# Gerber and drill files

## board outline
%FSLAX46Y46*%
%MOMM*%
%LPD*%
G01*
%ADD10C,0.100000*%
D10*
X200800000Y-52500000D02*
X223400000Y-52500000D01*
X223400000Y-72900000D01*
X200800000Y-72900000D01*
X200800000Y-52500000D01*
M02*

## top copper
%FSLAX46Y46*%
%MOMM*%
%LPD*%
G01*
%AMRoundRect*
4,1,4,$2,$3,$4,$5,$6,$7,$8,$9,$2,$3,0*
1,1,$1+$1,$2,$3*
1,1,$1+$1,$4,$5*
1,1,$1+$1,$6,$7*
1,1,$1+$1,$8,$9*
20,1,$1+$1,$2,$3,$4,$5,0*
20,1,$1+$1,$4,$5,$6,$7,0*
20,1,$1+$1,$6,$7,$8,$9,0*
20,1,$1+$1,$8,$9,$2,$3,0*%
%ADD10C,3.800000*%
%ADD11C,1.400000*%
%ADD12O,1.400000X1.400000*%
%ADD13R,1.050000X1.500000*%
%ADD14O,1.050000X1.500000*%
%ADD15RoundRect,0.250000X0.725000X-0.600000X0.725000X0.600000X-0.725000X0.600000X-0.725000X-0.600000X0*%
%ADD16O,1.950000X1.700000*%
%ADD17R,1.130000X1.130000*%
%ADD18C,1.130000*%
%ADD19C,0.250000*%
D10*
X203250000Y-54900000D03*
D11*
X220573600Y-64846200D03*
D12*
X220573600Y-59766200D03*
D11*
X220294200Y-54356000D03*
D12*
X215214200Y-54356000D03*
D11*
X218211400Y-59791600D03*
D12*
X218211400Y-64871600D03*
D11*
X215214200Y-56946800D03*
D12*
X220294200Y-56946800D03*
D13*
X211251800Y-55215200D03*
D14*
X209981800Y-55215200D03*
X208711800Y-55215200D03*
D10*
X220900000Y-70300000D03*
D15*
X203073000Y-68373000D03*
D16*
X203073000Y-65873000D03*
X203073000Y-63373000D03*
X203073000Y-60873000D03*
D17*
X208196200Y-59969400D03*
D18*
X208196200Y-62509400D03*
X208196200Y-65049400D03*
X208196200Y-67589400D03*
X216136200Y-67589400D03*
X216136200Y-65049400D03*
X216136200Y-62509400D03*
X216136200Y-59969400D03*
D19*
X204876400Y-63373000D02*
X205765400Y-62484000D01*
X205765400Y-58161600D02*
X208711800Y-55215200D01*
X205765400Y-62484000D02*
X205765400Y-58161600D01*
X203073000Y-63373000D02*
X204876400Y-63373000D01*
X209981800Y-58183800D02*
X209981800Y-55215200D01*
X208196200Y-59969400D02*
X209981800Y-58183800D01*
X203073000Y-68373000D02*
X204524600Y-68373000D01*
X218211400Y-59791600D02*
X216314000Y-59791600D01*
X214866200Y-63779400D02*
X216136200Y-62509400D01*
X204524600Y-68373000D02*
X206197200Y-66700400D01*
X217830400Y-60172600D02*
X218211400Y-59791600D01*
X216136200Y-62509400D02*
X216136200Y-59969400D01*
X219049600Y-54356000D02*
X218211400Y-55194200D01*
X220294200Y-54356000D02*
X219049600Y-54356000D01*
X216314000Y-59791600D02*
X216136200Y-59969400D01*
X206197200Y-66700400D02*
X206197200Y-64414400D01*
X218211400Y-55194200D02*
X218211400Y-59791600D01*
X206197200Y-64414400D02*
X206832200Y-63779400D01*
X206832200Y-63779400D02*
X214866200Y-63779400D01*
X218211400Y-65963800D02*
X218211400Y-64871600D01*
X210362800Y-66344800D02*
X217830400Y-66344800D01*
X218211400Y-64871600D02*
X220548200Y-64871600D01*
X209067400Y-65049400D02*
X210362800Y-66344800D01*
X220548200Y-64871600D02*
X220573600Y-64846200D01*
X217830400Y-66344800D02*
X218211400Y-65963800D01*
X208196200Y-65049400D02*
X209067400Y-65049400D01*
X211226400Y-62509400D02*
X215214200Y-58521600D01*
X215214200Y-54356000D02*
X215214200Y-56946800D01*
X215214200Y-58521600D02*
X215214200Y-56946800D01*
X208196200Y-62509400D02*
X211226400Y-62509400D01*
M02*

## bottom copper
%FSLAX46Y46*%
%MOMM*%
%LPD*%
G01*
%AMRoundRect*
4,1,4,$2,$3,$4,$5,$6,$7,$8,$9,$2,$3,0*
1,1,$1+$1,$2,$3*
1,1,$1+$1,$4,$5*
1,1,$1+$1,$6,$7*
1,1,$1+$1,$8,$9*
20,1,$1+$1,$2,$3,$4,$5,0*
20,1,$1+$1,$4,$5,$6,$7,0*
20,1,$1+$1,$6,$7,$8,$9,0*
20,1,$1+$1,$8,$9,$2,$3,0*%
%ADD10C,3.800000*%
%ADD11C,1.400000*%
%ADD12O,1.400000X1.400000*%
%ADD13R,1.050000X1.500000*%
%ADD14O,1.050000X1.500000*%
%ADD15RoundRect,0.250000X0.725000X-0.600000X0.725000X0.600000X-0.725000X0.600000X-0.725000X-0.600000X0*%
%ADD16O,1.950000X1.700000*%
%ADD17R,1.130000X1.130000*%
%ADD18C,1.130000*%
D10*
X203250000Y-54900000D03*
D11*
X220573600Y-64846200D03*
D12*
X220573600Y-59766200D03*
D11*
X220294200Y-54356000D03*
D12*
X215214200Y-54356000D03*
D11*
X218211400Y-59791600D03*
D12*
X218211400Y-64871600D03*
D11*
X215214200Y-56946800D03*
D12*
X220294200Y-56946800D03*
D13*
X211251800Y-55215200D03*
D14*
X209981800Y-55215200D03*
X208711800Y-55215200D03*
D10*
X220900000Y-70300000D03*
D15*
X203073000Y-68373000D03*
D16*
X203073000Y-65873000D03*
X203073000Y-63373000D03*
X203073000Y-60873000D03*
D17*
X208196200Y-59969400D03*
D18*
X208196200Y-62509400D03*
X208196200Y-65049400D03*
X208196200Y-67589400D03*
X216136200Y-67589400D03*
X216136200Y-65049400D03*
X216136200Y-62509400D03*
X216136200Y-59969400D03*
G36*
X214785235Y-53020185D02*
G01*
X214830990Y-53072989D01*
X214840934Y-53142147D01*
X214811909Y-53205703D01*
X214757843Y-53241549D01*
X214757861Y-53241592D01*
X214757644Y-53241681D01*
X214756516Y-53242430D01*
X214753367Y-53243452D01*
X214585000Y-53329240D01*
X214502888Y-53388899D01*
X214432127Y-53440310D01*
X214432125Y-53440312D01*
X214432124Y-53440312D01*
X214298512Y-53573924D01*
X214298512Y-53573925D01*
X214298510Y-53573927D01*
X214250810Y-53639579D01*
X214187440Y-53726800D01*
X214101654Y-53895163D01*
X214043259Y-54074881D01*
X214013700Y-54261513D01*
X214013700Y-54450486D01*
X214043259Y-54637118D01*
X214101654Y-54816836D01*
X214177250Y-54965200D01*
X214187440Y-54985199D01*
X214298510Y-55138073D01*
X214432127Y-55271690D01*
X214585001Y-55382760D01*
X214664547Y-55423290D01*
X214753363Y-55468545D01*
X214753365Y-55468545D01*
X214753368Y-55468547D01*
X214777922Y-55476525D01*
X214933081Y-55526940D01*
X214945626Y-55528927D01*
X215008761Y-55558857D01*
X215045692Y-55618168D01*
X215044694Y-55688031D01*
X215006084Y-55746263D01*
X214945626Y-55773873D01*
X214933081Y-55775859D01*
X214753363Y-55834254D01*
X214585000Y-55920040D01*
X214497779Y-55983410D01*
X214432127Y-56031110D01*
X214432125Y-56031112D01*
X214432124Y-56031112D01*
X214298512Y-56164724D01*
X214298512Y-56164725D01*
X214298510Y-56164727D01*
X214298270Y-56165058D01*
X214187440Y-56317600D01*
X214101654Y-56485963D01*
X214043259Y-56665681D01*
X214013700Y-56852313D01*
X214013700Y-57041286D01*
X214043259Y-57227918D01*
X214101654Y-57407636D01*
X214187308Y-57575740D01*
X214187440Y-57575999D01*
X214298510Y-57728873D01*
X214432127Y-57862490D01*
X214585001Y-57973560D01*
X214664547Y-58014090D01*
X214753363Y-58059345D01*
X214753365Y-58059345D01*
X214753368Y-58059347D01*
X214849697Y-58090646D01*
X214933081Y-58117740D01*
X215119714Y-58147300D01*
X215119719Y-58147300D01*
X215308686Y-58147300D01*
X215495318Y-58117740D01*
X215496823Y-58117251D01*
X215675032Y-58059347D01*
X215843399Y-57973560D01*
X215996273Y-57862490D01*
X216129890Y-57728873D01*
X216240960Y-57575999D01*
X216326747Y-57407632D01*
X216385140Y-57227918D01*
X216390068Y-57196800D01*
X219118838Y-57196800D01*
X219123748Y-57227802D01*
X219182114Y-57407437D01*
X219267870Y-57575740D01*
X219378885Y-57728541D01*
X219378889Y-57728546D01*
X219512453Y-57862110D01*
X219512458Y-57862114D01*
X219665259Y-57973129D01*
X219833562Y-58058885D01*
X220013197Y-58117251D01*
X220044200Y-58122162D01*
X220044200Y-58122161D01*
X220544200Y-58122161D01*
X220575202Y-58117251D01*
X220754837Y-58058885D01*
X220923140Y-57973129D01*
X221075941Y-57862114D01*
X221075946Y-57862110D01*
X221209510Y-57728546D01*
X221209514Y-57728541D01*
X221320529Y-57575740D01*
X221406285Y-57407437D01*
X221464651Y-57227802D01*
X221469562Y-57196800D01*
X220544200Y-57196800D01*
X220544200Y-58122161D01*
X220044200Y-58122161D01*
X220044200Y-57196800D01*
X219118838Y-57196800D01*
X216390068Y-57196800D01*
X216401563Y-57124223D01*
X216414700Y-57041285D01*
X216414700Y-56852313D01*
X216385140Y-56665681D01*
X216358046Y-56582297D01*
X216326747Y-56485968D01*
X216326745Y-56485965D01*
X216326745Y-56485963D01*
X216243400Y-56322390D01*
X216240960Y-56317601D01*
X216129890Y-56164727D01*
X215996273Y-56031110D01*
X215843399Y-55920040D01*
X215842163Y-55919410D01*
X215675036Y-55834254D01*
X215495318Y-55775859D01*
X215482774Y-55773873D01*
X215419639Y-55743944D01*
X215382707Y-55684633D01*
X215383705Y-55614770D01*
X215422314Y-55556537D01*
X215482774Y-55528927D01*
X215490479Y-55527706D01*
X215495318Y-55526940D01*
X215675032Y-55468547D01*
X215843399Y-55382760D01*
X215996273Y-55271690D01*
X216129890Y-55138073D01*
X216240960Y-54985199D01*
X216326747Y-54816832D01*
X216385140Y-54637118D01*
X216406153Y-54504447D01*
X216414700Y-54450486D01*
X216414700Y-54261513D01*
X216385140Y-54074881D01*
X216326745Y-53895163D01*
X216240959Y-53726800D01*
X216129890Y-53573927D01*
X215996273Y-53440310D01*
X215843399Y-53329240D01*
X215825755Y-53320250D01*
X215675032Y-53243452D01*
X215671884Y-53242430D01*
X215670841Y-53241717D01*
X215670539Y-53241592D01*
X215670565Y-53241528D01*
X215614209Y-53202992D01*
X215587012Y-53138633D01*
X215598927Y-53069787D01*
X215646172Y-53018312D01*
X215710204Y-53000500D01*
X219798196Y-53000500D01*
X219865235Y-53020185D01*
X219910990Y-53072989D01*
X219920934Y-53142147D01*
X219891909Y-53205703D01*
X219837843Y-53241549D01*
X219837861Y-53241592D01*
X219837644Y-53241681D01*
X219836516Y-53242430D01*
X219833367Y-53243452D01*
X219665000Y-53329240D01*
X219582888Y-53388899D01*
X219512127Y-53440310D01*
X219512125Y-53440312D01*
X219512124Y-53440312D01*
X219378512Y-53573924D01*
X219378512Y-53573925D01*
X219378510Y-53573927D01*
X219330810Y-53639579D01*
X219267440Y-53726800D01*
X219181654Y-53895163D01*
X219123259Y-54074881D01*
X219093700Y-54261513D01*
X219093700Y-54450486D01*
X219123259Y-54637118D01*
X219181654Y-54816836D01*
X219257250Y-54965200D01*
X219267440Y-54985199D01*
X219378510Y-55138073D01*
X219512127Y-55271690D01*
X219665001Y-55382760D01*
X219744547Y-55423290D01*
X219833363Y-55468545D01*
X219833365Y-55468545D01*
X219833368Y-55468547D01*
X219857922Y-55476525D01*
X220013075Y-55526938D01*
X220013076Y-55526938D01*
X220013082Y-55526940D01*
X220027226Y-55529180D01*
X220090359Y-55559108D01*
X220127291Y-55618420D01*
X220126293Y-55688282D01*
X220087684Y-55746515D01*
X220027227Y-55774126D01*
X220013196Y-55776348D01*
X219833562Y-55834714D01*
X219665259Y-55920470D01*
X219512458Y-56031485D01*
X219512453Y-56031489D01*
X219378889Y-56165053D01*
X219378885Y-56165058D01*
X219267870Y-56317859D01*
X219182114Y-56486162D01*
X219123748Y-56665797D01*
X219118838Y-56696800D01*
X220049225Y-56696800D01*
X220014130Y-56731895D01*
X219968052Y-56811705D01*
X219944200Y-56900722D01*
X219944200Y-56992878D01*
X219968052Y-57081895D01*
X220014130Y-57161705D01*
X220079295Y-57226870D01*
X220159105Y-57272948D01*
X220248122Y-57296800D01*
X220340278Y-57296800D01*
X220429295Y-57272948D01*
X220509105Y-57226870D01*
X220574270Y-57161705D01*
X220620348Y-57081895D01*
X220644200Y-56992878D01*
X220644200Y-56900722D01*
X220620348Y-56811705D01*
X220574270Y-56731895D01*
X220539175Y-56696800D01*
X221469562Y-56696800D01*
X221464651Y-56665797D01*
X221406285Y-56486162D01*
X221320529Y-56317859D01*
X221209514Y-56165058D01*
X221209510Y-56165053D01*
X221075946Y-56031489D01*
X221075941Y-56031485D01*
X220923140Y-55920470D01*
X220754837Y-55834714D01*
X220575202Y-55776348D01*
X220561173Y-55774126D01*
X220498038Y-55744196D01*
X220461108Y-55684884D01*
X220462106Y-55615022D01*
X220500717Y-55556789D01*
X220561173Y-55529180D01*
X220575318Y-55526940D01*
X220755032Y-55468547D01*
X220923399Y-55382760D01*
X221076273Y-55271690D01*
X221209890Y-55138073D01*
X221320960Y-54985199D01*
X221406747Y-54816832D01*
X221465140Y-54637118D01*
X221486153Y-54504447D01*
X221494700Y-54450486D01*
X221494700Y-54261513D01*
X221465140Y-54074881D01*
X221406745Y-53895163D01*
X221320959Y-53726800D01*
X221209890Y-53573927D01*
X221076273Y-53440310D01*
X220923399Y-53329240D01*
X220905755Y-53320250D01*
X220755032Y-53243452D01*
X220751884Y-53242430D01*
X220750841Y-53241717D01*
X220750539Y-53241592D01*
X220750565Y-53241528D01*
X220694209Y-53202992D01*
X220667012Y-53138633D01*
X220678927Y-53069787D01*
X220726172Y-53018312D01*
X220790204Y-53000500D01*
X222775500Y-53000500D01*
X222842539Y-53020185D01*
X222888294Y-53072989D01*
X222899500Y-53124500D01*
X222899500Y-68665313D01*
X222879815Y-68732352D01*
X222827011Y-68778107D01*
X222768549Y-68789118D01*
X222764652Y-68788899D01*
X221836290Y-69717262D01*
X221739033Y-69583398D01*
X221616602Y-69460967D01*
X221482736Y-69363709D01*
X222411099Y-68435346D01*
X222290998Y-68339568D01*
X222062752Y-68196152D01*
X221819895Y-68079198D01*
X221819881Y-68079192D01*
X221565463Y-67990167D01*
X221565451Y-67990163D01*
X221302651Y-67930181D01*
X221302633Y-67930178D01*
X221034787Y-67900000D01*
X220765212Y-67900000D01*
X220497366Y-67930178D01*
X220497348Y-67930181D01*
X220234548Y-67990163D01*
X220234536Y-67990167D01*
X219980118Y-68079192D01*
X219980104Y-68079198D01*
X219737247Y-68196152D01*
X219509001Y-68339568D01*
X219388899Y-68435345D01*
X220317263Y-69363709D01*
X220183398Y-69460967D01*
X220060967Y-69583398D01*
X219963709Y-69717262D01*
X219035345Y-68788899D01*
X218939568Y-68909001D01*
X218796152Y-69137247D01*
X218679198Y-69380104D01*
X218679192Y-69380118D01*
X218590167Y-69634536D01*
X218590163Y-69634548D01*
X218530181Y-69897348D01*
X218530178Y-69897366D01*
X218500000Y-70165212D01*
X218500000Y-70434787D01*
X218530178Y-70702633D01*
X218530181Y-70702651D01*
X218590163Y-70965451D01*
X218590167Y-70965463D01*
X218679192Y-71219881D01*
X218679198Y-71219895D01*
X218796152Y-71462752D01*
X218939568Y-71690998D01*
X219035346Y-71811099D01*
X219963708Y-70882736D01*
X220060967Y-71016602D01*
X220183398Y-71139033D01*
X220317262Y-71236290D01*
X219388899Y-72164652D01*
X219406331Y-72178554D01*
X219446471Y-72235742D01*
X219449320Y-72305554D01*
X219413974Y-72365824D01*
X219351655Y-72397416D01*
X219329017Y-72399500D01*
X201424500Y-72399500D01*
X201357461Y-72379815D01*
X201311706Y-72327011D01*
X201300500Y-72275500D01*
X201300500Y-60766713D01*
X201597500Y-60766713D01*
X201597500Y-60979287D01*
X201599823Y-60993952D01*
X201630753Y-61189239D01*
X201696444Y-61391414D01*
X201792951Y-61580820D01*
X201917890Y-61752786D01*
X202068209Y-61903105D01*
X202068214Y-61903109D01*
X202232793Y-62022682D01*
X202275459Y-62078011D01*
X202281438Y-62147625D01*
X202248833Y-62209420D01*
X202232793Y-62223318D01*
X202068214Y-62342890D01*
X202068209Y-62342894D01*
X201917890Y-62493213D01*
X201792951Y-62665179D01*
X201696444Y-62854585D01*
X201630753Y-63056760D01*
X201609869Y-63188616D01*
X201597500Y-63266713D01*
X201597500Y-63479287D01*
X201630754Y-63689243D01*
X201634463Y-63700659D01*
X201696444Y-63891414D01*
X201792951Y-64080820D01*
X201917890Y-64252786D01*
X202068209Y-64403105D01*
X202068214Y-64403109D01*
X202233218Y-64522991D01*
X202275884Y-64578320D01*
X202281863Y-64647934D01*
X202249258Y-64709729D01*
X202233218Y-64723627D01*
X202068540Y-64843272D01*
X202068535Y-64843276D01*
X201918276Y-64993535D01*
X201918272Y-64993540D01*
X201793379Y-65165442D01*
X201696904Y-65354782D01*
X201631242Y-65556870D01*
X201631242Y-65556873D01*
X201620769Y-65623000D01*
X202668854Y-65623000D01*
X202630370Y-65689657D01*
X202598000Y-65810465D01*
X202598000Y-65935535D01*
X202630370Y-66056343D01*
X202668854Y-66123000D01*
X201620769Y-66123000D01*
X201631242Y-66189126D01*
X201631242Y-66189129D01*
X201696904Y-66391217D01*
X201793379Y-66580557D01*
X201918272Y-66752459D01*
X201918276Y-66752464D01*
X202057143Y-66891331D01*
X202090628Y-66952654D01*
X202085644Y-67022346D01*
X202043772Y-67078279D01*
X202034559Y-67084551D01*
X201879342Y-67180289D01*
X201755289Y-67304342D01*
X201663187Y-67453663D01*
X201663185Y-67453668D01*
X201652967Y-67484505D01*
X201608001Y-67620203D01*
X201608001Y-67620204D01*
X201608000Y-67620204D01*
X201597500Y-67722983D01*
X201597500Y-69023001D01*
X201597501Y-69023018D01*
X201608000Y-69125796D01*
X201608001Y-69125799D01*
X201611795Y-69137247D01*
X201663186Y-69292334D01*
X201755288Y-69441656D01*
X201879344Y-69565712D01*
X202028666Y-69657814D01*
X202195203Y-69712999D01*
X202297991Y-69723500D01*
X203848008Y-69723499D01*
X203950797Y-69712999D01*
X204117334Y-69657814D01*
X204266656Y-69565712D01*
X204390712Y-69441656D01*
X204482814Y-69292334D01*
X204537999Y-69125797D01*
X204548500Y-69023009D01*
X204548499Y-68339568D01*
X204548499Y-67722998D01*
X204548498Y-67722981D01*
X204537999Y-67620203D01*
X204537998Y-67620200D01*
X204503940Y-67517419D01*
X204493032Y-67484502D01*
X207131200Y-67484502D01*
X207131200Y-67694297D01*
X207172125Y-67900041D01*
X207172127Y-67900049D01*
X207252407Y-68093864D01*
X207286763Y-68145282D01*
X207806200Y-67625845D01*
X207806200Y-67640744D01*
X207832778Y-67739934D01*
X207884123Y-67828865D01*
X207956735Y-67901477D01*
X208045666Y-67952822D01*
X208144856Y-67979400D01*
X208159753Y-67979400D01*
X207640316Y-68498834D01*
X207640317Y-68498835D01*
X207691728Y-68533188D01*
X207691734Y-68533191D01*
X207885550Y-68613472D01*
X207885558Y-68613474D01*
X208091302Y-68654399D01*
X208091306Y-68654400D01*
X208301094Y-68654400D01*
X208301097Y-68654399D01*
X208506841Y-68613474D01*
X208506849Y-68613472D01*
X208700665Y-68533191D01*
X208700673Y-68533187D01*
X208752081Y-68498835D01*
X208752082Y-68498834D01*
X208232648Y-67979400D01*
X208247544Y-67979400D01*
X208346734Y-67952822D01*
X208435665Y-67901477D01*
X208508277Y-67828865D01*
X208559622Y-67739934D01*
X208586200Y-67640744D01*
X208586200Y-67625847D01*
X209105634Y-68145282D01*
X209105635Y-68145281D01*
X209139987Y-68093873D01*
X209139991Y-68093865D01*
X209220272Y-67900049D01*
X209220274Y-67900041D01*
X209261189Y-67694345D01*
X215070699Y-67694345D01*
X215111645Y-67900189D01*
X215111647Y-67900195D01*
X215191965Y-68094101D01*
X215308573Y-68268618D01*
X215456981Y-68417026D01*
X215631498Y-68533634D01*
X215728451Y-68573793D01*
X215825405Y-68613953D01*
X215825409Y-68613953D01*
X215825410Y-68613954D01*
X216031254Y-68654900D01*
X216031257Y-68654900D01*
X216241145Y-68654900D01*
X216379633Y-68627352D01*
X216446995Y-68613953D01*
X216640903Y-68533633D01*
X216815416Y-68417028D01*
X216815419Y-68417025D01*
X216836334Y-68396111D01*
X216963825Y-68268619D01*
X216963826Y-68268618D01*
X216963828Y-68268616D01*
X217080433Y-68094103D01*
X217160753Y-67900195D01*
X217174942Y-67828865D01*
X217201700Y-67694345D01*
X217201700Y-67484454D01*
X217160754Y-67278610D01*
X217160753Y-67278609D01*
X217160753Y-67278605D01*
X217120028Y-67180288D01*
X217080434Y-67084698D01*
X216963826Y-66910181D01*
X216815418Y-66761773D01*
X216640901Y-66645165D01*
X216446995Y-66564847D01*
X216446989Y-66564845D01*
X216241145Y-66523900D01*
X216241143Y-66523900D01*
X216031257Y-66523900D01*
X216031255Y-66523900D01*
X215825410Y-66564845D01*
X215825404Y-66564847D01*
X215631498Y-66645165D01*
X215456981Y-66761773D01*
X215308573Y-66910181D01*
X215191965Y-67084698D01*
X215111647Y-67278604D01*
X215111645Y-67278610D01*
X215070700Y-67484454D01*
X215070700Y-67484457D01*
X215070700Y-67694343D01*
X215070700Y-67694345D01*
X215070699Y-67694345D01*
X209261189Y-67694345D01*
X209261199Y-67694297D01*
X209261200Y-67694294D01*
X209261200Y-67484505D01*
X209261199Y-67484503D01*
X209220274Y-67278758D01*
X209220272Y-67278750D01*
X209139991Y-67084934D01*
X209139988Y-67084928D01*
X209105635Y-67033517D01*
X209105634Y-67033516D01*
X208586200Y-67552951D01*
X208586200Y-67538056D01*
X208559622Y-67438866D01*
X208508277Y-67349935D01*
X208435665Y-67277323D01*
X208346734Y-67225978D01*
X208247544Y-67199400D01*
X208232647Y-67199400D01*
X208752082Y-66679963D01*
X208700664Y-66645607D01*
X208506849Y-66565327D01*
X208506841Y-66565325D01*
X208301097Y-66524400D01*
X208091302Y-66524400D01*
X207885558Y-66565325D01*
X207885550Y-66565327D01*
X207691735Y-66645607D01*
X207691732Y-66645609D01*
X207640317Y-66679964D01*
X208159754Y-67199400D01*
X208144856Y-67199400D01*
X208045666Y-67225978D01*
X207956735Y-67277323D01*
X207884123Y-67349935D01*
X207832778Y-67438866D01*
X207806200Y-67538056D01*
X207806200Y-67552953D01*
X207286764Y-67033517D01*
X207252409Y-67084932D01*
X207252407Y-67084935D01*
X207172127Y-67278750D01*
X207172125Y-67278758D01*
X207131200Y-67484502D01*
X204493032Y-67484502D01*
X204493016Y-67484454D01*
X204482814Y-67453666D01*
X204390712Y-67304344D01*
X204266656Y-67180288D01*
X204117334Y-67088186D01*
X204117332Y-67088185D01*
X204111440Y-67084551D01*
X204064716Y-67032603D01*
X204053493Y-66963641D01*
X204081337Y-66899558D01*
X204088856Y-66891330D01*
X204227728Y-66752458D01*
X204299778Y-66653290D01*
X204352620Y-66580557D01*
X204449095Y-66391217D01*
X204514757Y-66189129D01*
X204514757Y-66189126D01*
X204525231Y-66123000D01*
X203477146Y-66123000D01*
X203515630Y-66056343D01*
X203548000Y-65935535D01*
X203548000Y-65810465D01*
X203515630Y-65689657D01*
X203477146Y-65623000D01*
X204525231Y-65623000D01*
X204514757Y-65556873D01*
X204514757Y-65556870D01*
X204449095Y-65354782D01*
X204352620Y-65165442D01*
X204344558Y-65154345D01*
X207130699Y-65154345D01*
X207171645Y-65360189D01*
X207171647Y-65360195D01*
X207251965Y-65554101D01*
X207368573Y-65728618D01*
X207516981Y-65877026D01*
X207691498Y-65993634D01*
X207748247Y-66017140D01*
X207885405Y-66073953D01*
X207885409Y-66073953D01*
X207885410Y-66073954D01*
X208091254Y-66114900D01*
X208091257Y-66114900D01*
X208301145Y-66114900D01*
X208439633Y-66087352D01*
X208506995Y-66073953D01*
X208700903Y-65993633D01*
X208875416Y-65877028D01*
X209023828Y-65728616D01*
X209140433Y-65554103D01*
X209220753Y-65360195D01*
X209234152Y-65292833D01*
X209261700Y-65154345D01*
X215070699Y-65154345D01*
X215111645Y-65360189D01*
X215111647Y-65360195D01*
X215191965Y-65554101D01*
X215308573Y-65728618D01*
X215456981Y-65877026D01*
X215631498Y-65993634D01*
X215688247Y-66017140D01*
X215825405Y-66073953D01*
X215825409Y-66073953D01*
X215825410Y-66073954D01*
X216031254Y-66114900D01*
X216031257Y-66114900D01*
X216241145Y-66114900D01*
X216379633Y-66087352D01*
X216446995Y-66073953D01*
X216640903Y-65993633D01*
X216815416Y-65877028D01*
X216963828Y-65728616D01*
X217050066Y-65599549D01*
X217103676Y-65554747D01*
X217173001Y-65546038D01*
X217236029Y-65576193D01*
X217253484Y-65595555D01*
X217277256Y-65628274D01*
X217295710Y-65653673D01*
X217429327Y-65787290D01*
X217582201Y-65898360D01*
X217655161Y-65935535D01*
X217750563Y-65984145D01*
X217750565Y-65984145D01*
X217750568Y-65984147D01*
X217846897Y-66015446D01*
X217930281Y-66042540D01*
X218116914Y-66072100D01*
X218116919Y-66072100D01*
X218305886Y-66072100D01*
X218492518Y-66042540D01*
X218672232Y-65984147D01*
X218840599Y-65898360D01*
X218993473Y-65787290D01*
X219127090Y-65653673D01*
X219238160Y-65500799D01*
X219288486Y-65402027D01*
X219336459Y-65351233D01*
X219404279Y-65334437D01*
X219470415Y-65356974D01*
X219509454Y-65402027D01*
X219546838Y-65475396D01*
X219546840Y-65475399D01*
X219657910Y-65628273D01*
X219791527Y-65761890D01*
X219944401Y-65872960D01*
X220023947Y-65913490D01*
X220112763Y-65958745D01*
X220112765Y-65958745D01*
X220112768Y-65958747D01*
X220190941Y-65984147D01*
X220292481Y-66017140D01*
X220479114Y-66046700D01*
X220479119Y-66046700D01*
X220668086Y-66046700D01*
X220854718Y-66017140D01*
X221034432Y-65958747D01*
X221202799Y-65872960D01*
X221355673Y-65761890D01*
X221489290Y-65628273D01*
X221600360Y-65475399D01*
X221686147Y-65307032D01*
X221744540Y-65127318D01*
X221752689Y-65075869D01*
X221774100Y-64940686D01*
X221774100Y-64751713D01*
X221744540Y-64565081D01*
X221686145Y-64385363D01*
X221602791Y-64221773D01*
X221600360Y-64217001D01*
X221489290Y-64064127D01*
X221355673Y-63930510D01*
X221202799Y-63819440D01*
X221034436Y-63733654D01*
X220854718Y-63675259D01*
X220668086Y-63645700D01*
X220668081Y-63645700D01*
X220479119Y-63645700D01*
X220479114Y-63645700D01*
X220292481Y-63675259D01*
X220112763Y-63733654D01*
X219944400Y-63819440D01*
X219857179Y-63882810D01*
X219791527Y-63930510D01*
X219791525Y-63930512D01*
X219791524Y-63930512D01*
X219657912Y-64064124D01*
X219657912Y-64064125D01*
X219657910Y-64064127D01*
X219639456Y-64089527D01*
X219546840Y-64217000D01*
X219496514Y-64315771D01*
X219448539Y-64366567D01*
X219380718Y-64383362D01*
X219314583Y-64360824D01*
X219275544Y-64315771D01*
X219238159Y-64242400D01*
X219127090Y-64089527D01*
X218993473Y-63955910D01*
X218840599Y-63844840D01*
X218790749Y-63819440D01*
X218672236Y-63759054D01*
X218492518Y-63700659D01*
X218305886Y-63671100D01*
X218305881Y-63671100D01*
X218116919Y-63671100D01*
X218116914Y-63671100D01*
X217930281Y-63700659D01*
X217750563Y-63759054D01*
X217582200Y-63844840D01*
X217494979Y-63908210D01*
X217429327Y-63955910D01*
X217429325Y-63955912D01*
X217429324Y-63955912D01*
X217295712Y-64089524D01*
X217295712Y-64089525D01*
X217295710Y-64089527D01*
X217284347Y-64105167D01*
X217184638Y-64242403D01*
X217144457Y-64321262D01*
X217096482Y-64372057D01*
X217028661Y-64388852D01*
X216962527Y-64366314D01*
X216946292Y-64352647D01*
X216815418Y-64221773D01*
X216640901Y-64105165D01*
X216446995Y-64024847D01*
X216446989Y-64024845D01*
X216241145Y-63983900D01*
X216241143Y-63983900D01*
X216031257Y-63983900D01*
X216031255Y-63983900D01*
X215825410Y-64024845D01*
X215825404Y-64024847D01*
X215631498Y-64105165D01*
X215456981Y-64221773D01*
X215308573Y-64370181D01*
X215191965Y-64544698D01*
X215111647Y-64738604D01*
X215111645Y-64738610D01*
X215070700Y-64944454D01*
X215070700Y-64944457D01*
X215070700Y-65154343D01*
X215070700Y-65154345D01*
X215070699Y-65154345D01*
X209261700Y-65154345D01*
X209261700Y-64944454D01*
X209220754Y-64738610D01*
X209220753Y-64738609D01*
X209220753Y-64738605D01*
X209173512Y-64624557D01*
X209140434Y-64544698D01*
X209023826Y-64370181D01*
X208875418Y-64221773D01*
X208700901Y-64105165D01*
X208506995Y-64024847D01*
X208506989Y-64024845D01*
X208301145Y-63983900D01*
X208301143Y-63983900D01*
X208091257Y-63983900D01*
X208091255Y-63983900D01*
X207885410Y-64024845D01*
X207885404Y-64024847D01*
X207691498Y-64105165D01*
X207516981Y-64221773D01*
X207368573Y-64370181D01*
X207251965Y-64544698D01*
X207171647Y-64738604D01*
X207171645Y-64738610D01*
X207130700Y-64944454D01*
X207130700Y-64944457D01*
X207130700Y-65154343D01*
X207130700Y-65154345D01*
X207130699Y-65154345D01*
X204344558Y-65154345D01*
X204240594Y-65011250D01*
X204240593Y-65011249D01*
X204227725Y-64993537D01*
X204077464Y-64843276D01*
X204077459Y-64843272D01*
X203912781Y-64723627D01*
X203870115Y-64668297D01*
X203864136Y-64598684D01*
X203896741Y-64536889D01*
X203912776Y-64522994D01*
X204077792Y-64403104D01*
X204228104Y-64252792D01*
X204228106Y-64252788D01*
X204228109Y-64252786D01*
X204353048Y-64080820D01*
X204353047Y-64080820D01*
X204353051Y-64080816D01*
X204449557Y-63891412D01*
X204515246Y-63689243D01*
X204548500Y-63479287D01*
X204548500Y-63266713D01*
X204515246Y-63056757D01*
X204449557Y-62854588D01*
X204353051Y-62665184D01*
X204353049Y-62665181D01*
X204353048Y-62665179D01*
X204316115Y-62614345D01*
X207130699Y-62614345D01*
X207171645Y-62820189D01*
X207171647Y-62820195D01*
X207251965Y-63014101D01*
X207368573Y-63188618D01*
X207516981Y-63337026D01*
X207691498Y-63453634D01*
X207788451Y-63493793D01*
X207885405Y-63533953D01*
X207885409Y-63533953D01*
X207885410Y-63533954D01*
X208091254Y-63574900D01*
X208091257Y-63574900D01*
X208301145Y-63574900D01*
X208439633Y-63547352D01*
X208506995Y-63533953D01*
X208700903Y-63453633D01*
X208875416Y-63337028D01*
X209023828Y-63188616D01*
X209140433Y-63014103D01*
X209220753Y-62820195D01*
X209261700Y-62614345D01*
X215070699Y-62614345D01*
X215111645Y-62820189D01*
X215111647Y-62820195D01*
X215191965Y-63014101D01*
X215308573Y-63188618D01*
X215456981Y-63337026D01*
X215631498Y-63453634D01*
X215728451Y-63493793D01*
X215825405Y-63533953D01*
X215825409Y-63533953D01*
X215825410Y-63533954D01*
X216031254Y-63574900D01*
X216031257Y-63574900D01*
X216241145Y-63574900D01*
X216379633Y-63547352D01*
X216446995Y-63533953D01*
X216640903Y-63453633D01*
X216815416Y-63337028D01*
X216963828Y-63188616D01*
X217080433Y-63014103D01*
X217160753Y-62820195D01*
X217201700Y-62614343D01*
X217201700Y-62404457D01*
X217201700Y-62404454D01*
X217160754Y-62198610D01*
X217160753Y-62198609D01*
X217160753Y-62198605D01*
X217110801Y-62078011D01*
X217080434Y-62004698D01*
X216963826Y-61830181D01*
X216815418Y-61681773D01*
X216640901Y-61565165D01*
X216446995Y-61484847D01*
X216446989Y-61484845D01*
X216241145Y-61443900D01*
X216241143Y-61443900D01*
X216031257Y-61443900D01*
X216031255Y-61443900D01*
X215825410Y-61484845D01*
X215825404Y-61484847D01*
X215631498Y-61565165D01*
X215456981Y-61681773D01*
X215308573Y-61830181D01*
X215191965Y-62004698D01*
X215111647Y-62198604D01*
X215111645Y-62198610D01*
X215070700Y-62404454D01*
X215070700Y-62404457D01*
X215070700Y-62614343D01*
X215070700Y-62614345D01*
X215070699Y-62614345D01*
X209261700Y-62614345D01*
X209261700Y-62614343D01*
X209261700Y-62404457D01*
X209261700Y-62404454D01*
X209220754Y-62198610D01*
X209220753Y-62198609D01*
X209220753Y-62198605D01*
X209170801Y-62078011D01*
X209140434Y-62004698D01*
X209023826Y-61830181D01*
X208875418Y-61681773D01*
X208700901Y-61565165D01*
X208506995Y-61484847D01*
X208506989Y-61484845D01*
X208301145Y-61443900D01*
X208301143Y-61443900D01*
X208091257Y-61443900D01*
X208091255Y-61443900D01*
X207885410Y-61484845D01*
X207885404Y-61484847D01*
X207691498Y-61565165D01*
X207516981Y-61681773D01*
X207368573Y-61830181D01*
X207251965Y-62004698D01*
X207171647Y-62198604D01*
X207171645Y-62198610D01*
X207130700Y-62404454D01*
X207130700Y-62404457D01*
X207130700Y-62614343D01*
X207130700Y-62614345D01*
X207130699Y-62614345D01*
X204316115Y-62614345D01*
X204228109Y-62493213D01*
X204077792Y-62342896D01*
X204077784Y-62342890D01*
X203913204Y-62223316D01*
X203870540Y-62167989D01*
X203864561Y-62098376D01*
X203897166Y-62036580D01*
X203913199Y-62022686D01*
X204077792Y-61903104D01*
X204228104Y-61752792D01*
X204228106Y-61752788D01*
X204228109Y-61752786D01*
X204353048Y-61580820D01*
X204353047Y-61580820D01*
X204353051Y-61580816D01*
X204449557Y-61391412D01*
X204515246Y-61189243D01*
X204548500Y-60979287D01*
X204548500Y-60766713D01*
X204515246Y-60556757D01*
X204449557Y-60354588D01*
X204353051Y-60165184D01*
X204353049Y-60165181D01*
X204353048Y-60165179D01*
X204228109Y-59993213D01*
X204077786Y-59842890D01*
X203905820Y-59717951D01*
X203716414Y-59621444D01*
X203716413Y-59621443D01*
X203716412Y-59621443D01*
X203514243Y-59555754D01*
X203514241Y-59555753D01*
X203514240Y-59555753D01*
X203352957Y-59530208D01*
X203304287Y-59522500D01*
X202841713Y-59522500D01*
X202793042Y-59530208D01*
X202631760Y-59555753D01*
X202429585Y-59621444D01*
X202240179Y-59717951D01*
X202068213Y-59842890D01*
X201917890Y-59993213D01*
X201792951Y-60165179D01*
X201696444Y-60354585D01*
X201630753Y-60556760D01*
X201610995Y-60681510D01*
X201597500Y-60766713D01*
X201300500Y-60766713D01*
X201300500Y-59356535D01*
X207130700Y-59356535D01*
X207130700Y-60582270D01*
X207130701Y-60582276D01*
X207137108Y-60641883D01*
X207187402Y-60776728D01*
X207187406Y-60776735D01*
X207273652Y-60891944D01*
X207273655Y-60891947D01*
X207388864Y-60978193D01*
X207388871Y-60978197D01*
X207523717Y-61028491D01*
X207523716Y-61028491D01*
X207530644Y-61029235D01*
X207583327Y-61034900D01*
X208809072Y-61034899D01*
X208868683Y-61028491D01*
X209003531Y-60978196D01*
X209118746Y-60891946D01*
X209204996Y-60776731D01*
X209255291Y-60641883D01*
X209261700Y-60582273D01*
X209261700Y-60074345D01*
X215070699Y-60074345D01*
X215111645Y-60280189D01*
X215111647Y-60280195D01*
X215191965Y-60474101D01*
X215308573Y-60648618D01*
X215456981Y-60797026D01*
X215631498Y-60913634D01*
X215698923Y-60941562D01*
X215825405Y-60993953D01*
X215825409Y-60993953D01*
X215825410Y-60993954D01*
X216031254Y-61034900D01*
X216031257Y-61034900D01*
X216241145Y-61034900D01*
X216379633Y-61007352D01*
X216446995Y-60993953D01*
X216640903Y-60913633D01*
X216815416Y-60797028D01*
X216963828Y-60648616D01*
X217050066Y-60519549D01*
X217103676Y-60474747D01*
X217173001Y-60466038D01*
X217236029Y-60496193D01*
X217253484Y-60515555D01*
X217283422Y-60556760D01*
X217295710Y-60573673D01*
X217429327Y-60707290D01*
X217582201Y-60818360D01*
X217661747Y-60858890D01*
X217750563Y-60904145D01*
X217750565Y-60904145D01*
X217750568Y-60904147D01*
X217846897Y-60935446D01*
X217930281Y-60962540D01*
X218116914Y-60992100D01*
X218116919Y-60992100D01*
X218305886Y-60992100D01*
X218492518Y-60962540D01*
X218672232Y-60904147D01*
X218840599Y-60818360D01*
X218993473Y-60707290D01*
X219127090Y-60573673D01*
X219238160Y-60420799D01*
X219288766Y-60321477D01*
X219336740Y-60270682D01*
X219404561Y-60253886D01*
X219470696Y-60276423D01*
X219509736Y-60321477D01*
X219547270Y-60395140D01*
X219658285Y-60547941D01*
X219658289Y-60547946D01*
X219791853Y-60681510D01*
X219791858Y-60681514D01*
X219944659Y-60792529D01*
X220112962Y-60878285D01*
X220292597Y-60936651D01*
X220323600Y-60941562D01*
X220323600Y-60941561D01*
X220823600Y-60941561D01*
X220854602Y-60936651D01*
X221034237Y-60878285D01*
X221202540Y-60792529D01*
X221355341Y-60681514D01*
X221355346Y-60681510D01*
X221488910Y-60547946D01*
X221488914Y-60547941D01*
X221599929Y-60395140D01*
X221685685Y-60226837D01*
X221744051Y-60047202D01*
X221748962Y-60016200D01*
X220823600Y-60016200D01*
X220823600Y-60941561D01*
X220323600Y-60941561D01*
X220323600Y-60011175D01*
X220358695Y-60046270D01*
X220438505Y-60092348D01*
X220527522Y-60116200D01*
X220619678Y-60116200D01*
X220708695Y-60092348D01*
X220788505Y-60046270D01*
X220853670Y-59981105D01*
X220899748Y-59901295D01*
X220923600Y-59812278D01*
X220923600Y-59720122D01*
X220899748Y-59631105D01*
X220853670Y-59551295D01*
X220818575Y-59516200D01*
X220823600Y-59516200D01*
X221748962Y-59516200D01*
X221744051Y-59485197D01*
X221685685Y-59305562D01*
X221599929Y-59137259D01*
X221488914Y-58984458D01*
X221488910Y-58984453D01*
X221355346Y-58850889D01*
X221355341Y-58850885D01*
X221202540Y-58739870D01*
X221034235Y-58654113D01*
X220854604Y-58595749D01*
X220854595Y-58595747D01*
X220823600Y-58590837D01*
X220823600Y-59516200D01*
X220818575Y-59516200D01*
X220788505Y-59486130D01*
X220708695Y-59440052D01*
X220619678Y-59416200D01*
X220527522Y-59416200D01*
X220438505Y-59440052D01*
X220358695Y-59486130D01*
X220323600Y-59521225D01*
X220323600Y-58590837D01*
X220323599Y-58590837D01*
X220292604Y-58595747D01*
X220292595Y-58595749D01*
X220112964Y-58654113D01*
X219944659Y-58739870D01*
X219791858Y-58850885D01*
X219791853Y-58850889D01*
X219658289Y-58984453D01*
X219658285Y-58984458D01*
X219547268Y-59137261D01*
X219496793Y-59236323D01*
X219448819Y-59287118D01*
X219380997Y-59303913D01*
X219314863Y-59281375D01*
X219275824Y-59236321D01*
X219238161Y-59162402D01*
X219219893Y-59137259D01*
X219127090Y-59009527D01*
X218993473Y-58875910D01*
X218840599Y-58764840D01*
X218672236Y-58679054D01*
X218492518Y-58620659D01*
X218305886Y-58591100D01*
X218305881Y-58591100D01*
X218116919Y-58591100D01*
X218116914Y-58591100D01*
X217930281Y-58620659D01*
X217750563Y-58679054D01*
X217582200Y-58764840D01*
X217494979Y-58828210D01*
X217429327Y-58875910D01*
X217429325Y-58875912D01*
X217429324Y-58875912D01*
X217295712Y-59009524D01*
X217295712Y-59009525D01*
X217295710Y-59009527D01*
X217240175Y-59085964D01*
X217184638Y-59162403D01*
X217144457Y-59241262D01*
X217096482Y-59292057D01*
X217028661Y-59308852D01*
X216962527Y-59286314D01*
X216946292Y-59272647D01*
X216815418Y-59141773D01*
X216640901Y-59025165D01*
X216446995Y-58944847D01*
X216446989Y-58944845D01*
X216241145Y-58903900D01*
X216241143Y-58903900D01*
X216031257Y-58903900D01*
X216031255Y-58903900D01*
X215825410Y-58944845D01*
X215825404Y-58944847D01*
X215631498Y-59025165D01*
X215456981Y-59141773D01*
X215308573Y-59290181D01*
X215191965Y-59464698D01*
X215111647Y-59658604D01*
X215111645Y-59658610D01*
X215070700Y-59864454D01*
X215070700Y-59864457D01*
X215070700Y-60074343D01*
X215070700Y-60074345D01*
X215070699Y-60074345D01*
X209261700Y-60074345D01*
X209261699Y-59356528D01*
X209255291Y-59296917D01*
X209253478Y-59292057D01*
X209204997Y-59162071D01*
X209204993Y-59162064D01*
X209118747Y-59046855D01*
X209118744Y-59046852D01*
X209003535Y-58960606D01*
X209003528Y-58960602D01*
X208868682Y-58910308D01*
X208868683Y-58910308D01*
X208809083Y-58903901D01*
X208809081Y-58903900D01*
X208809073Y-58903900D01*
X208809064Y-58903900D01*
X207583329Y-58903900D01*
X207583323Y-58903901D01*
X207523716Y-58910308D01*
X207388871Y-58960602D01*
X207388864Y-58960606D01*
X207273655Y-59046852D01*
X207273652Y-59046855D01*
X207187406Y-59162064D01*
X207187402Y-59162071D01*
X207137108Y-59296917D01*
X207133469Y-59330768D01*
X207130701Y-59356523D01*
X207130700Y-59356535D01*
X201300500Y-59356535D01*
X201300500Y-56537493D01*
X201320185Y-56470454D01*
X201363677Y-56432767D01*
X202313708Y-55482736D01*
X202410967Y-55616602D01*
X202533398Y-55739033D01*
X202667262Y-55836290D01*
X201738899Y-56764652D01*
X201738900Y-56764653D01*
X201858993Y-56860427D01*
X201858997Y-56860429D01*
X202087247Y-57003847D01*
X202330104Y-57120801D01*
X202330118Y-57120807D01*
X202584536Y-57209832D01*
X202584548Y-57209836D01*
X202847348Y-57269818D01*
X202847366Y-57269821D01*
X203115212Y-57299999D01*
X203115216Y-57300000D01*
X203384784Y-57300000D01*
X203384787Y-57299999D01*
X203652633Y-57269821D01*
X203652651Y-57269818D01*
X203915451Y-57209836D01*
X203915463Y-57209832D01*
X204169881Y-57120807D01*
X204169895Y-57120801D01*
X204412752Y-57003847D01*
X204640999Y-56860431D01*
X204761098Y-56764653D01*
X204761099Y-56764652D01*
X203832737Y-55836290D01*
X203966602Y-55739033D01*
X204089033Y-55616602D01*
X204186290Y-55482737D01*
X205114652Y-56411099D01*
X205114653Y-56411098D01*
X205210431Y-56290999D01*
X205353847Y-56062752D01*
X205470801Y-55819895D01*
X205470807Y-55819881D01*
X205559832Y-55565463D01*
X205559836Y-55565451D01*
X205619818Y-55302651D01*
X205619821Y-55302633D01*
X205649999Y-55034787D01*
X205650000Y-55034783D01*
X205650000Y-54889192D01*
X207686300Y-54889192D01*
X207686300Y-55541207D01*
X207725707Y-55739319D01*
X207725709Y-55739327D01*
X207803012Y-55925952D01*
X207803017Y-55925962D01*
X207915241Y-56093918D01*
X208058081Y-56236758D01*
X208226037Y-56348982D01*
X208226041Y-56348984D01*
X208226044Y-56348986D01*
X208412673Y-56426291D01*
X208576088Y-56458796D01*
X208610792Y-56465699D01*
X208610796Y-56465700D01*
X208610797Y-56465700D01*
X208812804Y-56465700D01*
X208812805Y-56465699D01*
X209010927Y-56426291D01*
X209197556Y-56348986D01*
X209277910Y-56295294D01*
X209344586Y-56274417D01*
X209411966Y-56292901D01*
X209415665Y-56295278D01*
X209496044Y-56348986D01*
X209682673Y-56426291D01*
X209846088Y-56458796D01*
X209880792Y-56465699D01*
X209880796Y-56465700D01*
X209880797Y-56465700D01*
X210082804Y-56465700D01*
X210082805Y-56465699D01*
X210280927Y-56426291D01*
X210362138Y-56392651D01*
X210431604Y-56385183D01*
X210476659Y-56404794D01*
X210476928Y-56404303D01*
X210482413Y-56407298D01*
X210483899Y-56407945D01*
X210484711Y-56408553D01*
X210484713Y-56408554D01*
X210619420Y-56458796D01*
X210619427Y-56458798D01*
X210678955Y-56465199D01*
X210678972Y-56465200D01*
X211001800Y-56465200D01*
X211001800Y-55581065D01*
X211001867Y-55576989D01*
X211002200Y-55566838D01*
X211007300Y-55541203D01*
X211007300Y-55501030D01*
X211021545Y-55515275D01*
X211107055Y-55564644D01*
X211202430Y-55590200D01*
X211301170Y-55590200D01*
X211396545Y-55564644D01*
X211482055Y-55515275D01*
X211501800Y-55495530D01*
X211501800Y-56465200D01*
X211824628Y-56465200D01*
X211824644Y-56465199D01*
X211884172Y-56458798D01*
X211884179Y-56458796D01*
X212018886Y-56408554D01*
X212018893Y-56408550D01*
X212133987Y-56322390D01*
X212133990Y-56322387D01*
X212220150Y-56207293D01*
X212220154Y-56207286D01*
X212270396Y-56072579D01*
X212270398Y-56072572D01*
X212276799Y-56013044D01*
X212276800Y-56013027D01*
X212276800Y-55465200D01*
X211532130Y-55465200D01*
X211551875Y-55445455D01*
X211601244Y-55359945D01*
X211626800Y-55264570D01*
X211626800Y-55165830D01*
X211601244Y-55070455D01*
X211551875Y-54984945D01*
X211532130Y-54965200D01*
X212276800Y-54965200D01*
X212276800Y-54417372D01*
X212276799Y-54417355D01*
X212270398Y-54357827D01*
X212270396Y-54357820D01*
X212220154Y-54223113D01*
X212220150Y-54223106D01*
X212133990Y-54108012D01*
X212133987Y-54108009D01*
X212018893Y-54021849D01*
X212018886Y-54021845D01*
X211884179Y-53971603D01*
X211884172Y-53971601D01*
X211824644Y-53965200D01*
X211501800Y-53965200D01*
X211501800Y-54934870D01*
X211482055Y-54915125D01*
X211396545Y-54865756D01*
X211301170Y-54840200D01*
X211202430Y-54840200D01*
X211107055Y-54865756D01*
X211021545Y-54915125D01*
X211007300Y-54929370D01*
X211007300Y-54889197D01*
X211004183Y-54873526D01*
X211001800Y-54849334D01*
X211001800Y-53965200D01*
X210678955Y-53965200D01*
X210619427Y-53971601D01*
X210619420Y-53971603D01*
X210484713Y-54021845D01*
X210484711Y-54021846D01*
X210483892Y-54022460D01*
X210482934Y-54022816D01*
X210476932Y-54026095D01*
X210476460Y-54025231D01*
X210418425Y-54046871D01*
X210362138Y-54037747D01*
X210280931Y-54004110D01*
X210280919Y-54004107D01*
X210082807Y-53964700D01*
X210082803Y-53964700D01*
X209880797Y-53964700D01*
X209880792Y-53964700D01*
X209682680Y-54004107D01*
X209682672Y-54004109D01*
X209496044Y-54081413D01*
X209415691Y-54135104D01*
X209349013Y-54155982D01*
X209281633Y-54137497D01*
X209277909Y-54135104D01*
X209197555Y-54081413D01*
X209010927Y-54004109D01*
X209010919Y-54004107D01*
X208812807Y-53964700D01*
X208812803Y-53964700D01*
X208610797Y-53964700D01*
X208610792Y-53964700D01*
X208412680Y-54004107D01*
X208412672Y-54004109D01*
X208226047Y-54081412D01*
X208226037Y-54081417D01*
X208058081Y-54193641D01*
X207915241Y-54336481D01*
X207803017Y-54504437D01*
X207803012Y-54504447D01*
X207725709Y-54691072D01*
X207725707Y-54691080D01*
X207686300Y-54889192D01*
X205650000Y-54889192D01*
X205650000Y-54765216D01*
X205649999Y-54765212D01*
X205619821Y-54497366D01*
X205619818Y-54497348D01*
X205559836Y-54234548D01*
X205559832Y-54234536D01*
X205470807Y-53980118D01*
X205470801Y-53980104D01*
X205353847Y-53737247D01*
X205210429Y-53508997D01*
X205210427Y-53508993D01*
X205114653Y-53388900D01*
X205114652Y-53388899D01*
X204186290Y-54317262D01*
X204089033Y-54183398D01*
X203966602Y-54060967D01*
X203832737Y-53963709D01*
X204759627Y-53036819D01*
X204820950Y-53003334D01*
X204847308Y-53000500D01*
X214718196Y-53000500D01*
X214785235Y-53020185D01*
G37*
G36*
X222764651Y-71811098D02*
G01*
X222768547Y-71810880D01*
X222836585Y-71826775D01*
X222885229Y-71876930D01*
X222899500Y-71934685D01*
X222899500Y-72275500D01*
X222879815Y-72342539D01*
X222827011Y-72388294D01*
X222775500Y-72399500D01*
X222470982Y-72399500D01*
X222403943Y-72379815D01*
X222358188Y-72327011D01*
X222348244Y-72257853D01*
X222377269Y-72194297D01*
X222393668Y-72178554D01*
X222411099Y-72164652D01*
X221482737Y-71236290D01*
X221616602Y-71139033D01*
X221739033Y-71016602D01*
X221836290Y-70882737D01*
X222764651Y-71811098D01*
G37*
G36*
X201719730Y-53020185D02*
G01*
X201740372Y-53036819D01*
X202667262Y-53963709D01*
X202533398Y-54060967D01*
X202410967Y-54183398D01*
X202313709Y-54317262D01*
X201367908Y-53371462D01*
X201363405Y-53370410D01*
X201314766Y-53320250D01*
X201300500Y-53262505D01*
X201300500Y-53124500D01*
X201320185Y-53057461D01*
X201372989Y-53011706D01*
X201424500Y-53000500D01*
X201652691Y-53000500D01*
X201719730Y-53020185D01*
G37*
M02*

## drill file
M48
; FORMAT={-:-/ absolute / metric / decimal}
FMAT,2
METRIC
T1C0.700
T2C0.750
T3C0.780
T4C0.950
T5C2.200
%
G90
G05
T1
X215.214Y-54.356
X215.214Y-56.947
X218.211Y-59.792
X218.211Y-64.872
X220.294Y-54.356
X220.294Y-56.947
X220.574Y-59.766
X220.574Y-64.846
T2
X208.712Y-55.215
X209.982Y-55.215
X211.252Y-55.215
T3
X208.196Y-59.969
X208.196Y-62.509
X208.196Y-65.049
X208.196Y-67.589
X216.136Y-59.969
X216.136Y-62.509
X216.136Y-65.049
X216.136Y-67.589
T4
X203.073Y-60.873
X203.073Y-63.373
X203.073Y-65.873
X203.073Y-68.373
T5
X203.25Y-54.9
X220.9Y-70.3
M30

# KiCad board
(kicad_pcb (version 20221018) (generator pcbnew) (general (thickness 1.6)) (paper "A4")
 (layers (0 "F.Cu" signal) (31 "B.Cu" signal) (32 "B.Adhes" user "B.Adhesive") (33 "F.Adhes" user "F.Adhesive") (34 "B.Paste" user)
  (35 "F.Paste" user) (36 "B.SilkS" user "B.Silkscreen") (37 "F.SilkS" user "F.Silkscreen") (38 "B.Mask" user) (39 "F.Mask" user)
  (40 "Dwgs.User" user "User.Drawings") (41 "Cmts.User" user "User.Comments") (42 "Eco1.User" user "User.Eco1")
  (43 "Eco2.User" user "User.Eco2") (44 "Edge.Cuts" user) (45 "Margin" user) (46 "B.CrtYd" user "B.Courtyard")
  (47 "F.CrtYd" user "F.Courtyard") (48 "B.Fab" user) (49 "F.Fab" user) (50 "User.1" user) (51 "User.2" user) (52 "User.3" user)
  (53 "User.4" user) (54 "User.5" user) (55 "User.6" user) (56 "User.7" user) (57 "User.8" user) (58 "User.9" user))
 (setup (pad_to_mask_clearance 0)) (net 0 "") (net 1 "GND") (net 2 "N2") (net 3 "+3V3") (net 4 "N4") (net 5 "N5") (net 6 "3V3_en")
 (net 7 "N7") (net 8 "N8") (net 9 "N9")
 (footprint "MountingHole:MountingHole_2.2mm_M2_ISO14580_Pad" (layer "F.Cu") (at 203.25 54.9)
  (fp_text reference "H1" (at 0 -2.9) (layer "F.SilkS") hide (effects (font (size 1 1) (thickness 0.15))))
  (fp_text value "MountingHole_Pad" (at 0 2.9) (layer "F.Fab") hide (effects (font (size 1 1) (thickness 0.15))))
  (pad "1" thru_hole circle (at 0 0) (size 3.8 3.8) (drill 2.2) (layers "*.Cu" "*.Mask") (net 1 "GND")))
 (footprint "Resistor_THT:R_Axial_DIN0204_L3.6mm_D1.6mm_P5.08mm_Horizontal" (layer "F.Cu") (at 220.5736 64.8462 90)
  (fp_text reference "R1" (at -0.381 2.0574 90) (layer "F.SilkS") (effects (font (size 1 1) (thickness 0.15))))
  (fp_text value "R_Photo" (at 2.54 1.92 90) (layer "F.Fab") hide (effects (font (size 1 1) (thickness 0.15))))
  (pad "1" thru_hole circle (at 0 0 90) (size 1.4 1.4) (drill 0.7) (layers "*.Cu" "*.Mask") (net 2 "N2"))
  (pad "2" thru_hole oval (at 5.08 0 90) (size 1.4 1.4) (drill 0.7) (layers "*.Cu" "*.Mask") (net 1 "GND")))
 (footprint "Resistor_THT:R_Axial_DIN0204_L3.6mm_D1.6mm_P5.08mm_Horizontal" (layer "F.Cu") (at 220.2942 54.356 180)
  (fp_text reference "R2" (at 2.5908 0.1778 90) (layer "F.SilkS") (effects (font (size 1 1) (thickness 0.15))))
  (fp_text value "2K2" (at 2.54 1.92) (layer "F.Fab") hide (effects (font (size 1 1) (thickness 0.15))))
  (pad "1" thru_hole circle (at 0 0 180) (size 1.4 1.4) (drill 0.7) (layers "*.Cu" "*.Mask") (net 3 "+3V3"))
  (pad "2" thru_hole oval (at 5.08 0 180) (size 1.4 1.4) (drill 0.7) (layers "*.Cu" "*.Mask") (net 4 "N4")))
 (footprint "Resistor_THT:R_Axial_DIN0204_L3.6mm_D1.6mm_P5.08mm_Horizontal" (layer "F.Cu") (at 218.2114 59.7916 -90)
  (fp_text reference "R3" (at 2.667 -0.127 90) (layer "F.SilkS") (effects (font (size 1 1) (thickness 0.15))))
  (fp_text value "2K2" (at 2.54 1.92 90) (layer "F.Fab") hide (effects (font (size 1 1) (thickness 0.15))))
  (pad "1" thru_hole circle (at 0 0 270) (size 1.4 1.4) (drill 0.7) (layers "*.Cu" "*.Mask") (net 3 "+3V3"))
  (pad "2" thru_hole oval (at 5.08 0 270) (size 1.4 1.4) (drill 0.7) (layers "*.Cu" "*.Mask") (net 2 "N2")))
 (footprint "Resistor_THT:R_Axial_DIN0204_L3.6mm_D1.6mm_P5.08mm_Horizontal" (layer "F.Cu") (at 215.2142 56.9468)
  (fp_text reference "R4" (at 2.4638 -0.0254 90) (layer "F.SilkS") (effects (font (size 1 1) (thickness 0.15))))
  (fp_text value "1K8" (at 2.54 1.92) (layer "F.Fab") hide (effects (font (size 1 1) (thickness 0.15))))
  (pad "1" thru_hole circle (at 0 0) (size 1.4 1.4) (drill 0.7) (layers "*.Cu" "*.Mask") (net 4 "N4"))
  (pad "2" thru_hole oval (at 5.08 0) (size 1.4 1.4) (drill 0.7) (layers "*.Cu" "*.Mask") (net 1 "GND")))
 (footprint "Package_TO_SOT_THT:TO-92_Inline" (layer "F.Cu") (at 211.2518 55.2152 180)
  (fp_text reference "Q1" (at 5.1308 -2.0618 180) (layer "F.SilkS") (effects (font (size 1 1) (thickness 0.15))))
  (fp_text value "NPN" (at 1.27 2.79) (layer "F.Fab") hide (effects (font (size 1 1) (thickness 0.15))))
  (pad "1" thru_hole rect (at 0 0 180) (size 1.05 1.5) (drill 0.75) (layers "*.Cu" "*.Mask") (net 1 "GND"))
  (pad "2" thru_hole oval (at 1.27 0 180) (size 1.05 1.5) (drill 0.75) (layers "*.Cu" "*.Mask") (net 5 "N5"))
  (pad "3" thru_hole oval (at 2.54 0 180) (size 1.05 1.5) (drill 0.75) (layers "*.Cu" "*.Mask") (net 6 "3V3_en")))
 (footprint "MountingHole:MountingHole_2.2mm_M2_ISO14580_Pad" (layer "F.Cu") (at 220.9 70.3)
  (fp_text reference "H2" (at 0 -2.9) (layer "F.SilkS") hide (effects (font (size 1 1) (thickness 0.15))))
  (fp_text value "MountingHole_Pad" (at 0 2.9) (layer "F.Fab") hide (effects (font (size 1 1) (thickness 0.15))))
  (pad "1" thru_hole circle (at 0 0) (size 3.8 3.8) (drill 2.2) (layers "*.Cu" "*.Mask") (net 1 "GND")))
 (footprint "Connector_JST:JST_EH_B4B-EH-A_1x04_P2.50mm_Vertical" (layer "F.Cu") (at 203.073 68.373 90)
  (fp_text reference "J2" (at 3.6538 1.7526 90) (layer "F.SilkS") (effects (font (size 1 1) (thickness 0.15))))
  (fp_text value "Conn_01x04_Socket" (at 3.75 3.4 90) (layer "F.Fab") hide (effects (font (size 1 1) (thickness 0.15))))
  (pad "1" thru_hole roundrect (at 0 0 90) (size 1.7 1.95) (drill 0.95) (layers "*.Cu" "*.Mask") (roundrect_rratio 0.1470588235)
   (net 3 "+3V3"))
  (pad "2" thru_hole oval (at 2.5 0 90) (size 1.7 1.95) (drill 0.95) (layers "*.Cu" "*.Mask") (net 1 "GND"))
  (pad "3" thru_hole oval (at 5 0 90) (size 1.7 1.95) (drill 0.95) (layers "*.Cu" "*.Mask") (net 6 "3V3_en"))
  (pad "4" thru_hole oval (at 7.5 0 90) (size 1.7 1.95) (drill 0.95) (layers "*.Cu" "*.Mask") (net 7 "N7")))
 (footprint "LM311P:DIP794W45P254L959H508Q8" (layer "F.Cu") (at 212.1662 63.7794)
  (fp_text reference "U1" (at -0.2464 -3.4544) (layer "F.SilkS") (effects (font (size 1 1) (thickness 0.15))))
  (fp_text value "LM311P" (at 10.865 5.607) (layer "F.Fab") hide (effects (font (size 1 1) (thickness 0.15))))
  (pad "1" thru_hole rect (at -3.97 -3.81) (size 1.13 1.13) (drill 0.78) (layers "*.Cu" "*.Mask") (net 5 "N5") (solder_mask_margin 0.102))
  (pad "2" thru_hole circle (at -3.97 -1.27) (size 1.13 1.13) (drill 0.78) (layers "*.Cu" "*.Mask") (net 4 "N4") (solder_mask_margin 0.102))
  (pad "3" thru_hole circle (at -3.97 1.27) (size 1.13 1.13) (drill 0.78) (layers "*.Cu" "*.Mask") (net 2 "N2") (solder_mask_margin 0.102))
  (pad "4" thru_hole circle (at -3.97 3.81) (size 1.13 1.13) (drill 0.78) (layers "*.Cu" "*.Mask") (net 1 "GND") (solder_mask_margin 0.102))
  (pad "5" thru_hole circle (at 3.97 3.81) (size 1.13 1.13) (drill 0.78) (layers "*.Cu" "*.Mask") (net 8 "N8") (solder_mask_margin 0.102))
  (pad "6" thru_hole circle (at 3.97 1.27) (size 1.13 1.13) (drill 0.78) (layers "*.Cu" "*.Mask") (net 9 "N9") (solder_mask_margin 0.102))
  (pad "7" thru_hole circle (at 3.97 -1.27) (size 1.13 1.13) (drill 0.78) (layers "*.Cu" "*.Mask") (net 3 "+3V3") (solder_mask_margin 0.102))
  (pad "8" thru_hole circle (at 3.97 -3.81) (size 1.13 1.13) (drill 0.78) (layers "*.Cu" "*.Mask") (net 3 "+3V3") (solder_mask_margin 0.102)))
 (gr_rect (start 200.8 52.5) (end 223.4 72.9) (stroke (width 0.1) (type default)) (fill none) (layer "Edge.Cuts"))
 (segment (start 204.8764 63.373) (end 205.7654 62.484) (width 0.25) (layer "F.Cu") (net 6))
 (segment (start 205.7654 58.1616) (end 208.7118 55.2152) (width 0.25) (layer "F.Cu") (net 6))
 (segment (start 205.7654 62.484) (end 205.7654 58.1616) (width 0.25) (layer "F.Cu") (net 6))
 (segment (start 203.073 63.373) (end 204.8764 63.373) (width 0.25) (layer "F.Cu") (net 6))
 (segment (start 209.9818 58.1838) (end 209.9818 55.2152) (width 0.25) (layer "F.Cu") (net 5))
 (segment (start 208.1962 59.9694) (end 209.9818 58.1838) (width 0.25) (layer "F.Cu") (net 5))
 (segment (start 203.073 68.373) (end 204.5246 68.373) (width 0.25) (layer "F.Cu") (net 3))
 (segment (start 218.2114 59.7916) (end 216.314 59.7916) (width 0.25) (layer "F.Cu") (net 3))
 (segment (start 214.8662 63.7794) (end 216.1362 62.5094) (width 0.25) (layer "F.Cu") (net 3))
 (segment (start 204.5246 68.373) (end 206.1972 66.7004) (width 0.25) (layer "F.Cu") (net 3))
 (segment (start 217.8304 60.1726) (end 218.2114 59.7916) (width 0.25) (layer "F.Cu") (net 3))
 (segment (start 216.1362 62.5094) (end 216.1362 59.9694) (width 0.25) (layer "F.Cu") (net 3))
 (segment (start 219.0496 54.356) (end 218.2114 55.1942) (width 0.25) (layer "F.Cu") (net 3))
 (segment (start 220.2942 54.356) (end 219.0496 54.356) (width 0.25) (layer "F.Cu") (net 3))
 (segment (start 216.314 59.7916) (end 216.1362 59.9694) (width 0.25) (layer "F.Cu") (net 3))
 (segment (start 206.1972 66.7004) (end 206.1972 64.4144) (width 0.25) (layer "F.Cu") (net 3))
 (segment (start 218.2114 55.1942) (end 218.2114 59.7916) (width 0.25) (layer "F.Cu") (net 3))
 (segment (start 206.1972 64.4144) (end 206.8322 63.7794) (width 0.25) (layer "F.Cu") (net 3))
 (segment (start 206.8322 63.7794) (end 214.8662 63.7794) (width 0.25) (layer "F.Cu") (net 3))
 (segment (start 218.2114 65.9638) (end 218.2114 64.8716) (width 0.25) (layer "F.Cu") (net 2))
 (segment (start 210.3628 66.3448) (end 217.8304 66.3448) (width 0.25) (layer "F.Cu") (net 2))
 (segment (start 218.2114 64.8716) (end 220.5482 64.8716) (width 0.25) (layer "F.Cu") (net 2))
 (segment (start 209.0674 65.0494) (end 210.3628 66.3448) (width 0.25) (layer "F.Cu") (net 2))
 (segment (start 220.5482 64.8716) (end 220.5736 64.8462) (width 0.25) (layer "F.Cu") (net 2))
 (segment (start 217.8304 66.3448) (end 218.2114 65.9638) (width 0.25) (layer "F.Cu") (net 2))
 (segment (start 208.1962 65.0494) (end 209.0674 65.0494) (width 0.25) (layer "F.Cu") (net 2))
 (segment (start 211.2264 62.5094) (end 215.2142 58.5216) (width 0.25) (layer "F.Cu") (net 4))
 (segment (start 215.2142 54.356) (end 215.2142 56.9468) (width 0.25) (layer "F.Cu") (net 4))
 (segment (start 215.2142 58.5216) (end 215.2142 56.9468) (width 0.25) (layer "F.Cu") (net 4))
 (segment (start 208.1962 62.5094) (end 211.2264 62.5094) (width 0.25) (layer "F.Cu") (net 4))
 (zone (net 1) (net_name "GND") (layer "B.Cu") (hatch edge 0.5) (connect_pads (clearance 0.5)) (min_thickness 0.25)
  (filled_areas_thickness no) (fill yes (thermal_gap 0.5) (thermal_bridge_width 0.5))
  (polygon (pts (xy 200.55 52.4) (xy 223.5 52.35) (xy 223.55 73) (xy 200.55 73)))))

